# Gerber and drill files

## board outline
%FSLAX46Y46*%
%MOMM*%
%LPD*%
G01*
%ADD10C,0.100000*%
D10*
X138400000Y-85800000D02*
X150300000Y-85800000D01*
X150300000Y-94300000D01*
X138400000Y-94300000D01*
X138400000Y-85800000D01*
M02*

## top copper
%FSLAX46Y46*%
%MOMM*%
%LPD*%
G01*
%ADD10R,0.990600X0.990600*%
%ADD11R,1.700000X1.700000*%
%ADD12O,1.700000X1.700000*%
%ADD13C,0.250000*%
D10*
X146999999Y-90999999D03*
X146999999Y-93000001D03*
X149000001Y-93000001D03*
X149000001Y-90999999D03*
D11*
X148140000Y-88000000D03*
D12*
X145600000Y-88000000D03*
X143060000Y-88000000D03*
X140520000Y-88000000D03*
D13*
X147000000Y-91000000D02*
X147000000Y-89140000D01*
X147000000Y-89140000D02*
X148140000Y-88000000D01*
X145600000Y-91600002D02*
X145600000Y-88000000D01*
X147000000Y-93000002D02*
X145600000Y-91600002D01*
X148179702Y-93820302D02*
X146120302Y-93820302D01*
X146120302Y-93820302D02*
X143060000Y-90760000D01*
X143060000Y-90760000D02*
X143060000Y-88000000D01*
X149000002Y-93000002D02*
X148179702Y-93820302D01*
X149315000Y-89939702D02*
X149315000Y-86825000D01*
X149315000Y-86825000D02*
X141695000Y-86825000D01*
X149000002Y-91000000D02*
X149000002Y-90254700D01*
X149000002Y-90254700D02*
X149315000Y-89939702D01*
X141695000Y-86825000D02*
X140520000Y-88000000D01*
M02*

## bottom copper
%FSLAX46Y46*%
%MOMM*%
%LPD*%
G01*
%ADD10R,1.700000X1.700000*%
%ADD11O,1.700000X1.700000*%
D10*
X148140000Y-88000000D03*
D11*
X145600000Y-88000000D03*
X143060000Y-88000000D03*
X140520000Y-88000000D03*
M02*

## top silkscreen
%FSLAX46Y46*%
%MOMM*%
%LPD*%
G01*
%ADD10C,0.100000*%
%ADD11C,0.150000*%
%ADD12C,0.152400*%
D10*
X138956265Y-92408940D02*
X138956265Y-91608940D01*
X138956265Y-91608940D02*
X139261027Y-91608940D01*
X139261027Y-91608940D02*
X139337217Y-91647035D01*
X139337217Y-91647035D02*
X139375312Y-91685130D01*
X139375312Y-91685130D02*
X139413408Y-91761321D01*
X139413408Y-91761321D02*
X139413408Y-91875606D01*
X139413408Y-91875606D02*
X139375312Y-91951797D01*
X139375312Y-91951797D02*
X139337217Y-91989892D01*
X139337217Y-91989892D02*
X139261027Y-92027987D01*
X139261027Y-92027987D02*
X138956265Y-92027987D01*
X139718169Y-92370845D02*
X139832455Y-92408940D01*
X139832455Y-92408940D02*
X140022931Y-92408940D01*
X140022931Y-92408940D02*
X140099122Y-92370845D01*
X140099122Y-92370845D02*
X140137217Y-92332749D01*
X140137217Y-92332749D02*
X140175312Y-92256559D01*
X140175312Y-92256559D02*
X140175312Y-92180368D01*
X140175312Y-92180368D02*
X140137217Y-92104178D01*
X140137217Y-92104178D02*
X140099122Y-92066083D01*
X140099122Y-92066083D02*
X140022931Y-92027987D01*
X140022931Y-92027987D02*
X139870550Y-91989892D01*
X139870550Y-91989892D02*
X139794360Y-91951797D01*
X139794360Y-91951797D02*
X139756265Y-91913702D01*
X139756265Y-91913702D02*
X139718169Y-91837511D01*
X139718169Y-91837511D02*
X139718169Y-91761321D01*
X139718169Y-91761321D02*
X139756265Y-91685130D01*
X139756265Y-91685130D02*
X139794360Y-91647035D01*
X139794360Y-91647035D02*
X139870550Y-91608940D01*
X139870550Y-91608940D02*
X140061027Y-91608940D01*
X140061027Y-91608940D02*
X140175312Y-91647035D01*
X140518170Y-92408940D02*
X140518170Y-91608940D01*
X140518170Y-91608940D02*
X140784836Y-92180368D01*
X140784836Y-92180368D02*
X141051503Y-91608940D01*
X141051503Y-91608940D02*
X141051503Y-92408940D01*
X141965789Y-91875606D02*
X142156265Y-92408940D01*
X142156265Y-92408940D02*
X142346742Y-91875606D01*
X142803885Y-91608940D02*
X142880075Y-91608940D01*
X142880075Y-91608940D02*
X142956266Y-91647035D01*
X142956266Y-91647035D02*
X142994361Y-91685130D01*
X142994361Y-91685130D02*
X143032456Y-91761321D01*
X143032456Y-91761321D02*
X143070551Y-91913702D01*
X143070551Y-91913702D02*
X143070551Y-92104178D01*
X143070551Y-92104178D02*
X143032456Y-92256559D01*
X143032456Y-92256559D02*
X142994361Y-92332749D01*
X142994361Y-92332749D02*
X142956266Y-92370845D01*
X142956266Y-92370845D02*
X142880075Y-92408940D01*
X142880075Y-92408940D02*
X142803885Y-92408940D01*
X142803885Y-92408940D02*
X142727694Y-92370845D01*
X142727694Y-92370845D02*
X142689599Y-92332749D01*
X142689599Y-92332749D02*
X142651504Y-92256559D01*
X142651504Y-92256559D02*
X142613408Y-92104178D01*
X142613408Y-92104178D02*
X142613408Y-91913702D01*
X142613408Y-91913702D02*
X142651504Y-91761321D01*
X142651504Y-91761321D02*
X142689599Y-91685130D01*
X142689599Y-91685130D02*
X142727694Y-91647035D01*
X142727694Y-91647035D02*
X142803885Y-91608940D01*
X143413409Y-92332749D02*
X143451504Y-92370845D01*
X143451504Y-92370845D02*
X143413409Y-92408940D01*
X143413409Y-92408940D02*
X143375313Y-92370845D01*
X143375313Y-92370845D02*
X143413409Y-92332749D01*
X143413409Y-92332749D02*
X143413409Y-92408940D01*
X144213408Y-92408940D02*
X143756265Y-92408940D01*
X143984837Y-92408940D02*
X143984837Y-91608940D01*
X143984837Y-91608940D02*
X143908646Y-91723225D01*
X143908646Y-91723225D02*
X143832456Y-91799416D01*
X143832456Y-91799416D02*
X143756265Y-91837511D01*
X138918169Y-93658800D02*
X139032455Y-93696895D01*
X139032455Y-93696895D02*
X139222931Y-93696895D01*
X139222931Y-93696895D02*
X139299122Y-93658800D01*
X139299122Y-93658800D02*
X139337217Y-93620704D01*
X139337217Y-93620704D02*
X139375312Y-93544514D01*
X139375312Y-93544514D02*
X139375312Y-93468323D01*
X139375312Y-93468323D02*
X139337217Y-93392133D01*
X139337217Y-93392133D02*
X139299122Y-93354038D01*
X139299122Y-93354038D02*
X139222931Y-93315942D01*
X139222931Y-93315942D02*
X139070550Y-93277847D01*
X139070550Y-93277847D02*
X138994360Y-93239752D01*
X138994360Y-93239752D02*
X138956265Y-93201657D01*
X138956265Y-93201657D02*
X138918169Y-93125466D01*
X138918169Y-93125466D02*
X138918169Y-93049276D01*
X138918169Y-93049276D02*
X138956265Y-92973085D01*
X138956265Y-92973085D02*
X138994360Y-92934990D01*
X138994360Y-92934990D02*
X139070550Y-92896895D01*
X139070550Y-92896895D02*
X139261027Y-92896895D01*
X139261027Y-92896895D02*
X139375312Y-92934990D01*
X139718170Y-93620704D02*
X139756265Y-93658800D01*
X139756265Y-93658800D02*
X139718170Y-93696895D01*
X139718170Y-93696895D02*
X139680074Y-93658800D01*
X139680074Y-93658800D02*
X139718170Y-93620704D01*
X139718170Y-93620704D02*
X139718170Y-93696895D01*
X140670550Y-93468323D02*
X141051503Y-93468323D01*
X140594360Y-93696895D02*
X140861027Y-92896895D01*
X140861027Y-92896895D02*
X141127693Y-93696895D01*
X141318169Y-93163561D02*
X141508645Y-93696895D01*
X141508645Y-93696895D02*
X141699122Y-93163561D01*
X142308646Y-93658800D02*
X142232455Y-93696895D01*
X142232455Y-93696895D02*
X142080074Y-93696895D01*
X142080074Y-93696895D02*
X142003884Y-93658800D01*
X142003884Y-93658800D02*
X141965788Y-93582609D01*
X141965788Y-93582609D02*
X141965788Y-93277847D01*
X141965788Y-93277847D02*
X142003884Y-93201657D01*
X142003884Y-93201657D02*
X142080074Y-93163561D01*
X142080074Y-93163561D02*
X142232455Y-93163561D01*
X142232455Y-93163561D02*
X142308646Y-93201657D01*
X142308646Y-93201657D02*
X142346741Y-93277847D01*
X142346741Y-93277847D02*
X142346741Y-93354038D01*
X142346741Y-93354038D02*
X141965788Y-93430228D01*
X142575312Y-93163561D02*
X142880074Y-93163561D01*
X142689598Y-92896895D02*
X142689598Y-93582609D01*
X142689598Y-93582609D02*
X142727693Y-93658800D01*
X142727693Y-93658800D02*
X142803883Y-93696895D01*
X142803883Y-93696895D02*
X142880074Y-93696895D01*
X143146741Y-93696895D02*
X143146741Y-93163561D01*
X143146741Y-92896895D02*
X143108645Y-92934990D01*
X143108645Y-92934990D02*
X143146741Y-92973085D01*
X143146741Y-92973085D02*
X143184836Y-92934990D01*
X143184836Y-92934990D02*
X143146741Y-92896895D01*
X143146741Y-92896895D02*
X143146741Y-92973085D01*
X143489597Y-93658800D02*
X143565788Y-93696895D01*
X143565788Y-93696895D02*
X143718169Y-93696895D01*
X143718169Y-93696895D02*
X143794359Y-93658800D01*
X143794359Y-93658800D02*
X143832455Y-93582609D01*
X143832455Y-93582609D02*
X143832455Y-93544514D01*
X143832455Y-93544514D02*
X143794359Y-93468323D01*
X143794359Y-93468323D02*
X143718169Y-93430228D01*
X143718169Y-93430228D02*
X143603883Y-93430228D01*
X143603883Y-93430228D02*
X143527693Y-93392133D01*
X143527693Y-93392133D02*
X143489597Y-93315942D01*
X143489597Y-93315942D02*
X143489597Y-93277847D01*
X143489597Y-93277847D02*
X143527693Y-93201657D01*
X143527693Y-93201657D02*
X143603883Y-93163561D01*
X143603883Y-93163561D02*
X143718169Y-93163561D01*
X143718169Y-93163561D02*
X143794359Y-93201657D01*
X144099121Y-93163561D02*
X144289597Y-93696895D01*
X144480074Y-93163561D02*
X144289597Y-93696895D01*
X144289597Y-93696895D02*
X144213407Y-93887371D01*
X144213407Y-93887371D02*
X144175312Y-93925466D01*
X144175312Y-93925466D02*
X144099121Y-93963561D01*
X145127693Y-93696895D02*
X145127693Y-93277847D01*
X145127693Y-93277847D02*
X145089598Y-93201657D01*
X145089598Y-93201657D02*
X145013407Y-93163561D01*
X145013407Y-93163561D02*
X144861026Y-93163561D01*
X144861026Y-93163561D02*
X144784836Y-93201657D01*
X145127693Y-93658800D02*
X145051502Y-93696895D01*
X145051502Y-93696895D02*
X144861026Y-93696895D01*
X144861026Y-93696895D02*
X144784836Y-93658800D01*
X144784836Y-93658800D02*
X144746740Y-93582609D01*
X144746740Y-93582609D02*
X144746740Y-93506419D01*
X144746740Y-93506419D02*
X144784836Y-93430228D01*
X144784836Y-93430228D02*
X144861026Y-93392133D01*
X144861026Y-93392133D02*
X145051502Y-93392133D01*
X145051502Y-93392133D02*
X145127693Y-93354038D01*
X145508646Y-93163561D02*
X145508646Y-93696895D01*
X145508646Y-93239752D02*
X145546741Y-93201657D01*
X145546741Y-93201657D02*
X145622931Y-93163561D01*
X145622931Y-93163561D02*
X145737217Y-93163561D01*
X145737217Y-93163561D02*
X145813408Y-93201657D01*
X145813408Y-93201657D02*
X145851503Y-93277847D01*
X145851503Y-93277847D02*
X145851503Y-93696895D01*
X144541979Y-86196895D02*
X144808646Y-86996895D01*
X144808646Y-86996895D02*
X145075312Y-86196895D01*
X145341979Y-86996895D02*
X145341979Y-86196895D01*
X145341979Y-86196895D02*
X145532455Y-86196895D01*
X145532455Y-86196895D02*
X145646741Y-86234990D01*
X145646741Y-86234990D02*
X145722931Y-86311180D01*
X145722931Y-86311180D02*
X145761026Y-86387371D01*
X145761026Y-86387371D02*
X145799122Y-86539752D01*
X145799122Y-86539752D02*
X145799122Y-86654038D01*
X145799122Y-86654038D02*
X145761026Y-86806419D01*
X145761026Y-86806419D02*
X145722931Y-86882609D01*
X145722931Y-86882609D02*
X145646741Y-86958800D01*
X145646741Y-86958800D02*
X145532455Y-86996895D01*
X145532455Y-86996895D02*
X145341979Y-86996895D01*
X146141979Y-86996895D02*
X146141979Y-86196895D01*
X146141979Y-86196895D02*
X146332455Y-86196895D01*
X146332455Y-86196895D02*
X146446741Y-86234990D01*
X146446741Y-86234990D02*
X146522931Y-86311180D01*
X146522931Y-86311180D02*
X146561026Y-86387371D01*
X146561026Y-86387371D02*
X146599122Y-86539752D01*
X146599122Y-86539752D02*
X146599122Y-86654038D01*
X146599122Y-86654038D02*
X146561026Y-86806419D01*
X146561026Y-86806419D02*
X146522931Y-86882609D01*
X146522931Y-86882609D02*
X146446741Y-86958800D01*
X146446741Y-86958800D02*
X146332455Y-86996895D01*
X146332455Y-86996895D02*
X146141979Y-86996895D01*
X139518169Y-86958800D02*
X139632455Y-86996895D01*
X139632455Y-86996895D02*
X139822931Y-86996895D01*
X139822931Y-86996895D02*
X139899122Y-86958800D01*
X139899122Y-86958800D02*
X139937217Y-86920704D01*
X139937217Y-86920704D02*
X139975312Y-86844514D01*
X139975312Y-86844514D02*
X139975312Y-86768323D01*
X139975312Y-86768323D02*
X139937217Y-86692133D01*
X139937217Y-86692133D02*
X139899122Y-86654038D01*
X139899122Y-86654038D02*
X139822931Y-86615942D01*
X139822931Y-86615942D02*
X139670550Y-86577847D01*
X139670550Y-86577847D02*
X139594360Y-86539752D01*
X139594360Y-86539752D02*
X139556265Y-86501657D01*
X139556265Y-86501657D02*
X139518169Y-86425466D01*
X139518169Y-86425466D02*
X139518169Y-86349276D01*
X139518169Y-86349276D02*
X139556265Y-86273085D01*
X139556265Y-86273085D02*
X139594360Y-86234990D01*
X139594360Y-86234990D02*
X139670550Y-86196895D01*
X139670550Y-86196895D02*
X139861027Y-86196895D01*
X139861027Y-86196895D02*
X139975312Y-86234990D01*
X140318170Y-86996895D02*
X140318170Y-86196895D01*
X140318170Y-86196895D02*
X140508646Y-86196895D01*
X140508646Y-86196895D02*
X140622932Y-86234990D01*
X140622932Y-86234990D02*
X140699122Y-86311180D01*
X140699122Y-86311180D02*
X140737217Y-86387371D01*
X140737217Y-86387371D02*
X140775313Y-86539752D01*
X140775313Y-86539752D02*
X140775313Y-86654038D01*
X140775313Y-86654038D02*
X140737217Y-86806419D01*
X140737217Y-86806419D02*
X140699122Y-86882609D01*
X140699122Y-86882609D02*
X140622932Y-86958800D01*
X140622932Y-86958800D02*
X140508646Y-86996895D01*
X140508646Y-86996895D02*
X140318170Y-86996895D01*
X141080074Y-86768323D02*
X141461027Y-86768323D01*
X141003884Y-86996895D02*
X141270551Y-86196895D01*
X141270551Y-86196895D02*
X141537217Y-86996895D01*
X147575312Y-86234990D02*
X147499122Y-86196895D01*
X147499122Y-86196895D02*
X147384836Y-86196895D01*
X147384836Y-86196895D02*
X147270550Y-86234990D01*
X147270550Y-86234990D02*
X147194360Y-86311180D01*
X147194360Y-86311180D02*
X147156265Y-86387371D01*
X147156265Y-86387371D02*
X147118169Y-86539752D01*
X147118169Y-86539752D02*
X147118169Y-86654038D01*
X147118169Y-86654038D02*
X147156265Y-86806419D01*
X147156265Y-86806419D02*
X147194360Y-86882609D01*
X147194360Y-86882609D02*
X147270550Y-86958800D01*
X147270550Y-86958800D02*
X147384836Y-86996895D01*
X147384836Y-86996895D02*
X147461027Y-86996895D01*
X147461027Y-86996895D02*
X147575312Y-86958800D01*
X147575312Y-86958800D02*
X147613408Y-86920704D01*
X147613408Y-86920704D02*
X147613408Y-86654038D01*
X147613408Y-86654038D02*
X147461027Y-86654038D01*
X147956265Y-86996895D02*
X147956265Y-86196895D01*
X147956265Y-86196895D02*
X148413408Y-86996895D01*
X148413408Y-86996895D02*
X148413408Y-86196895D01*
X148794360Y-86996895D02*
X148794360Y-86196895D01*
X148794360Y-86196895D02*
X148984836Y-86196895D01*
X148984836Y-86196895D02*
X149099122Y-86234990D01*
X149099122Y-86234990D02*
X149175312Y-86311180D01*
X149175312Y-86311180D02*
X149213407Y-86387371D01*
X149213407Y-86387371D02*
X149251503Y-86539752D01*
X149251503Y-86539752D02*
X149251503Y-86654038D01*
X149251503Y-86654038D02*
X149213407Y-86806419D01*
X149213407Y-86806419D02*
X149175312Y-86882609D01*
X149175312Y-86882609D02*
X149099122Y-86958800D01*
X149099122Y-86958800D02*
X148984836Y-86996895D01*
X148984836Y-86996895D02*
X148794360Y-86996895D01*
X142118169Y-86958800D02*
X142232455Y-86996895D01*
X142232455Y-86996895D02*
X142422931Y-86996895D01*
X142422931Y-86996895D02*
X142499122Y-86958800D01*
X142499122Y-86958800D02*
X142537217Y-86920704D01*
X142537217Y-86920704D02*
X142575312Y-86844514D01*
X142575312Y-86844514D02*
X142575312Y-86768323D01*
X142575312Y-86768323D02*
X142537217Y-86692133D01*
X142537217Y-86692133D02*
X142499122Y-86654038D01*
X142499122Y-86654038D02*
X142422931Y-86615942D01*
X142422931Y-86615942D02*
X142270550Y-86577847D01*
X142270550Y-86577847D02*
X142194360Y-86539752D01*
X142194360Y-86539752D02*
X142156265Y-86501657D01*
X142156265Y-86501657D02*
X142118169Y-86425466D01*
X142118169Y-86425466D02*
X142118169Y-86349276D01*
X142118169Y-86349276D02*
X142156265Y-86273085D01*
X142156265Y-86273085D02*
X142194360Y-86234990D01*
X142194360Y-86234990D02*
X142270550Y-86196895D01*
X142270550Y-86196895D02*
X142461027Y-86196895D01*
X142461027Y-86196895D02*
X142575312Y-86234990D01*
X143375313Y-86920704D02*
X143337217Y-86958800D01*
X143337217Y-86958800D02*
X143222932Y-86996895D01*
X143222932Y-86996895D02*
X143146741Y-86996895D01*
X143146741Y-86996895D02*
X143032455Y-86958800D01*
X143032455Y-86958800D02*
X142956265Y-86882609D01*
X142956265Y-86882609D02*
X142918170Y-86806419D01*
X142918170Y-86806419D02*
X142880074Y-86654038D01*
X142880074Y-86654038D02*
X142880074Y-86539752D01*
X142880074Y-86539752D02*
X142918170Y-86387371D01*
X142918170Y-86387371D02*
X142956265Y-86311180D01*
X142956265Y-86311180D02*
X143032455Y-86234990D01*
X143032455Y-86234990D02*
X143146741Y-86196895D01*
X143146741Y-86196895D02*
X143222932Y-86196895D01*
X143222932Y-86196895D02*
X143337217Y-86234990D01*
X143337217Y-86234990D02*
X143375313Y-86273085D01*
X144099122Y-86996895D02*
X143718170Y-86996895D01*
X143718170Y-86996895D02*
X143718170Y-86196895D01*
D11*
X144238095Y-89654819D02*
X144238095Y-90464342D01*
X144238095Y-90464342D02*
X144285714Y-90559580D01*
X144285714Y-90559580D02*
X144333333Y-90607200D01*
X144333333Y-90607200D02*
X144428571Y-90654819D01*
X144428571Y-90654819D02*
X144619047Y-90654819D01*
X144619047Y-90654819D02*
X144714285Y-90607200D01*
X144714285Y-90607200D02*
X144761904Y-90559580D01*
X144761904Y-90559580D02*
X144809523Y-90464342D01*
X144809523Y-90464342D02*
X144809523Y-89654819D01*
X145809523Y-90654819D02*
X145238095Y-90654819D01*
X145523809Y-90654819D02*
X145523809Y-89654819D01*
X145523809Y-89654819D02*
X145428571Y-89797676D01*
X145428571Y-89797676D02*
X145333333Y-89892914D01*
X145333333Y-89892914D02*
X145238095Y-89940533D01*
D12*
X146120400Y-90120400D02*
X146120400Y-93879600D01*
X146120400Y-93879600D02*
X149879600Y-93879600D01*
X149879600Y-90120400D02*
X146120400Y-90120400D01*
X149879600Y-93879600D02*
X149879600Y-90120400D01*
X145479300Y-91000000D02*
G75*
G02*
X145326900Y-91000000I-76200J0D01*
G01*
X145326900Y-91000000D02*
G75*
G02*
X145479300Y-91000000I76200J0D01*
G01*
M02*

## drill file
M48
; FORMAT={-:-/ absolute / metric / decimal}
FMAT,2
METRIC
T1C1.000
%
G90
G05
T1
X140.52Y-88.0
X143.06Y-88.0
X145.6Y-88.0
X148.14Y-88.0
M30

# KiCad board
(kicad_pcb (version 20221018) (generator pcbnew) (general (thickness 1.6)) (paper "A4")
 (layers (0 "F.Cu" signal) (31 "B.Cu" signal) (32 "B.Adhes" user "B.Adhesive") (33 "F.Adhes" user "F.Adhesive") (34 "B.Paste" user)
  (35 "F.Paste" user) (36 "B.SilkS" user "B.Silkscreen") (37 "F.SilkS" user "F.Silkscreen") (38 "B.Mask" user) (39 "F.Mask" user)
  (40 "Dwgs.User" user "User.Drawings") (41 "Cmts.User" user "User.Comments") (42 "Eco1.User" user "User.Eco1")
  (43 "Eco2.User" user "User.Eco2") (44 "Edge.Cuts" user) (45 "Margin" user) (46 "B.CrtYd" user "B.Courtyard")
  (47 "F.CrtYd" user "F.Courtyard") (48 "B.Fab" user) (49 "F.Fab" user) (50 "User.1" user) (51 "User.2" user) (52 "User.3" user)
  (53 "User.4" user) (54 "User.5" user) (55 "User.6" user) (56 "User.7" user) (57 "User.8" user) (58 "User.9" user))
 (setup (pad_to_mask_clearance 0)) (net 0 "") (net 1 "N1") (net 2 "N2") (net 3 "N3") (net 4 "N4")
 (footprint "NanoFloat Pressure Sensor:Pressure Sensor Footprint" (layer "F.Cu") (at 148 92)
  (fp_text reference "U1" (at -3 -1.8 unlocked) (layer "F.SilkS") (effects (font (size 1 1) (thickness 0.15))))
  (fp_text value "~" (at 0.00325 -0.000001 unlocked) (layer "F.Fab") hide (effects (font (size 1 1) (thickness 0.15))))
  (fp_line (start -1.8796 -1.8796) (end -1.8796 1.8796) (stroke (width 0.1524) (type solid)) (layer "F.SilkS"))
  (fp_line (start -1.8796 1.8796) (end 1.8796 1.8796) (stroke (width 0.1524) (type solid)) (layer "F.SilkS"))
  (fp_line (start 1.8796 -1.8796) (end -1.8796 -1.8796) (stroke (width 0.1524) (type solid)) (layer "F.SilkS"))
  (fp_line (start 1.8796 1.8796) (end 1.8796 -1.8796) (stroke (width 0.1524) (type solid)) (layer "F.SilkS"))
  (fp_circle (center -2.5969 -1) (end -2.5207 -1) (stroke (width 0.1524) (type solid)) (fill none) (layer "F.SilkS"))
  (pad "1" smd rect (at -1.000001 -1.000001) (size 0.9906 0.9906) (layers "F.Cu" "F.Paste" "F.Mask") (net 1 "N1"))
  (pad "2" smd rect (at -1.000001 1.000001) (size 0.9906 0.9906) (layers "F.Cu" "F.Paste" "F.Mask") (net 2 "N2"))
  (pad "3" smd rect (at 1.000001 1.000001) (size 0.9906 0.9906) (layers "F.Cu" "F.Paste" "F.Mask") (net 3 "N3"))
  (pad "4" smd rect (at 1.000001 -1.000001) (size 0.9906 0.9906) (layers "F.Cu" "F.Paste" "F.Mask") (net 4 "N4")))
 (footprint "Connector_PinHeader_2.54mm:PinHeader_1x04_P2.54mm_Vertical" (layer "B.Cu") (at 148.14 88 90)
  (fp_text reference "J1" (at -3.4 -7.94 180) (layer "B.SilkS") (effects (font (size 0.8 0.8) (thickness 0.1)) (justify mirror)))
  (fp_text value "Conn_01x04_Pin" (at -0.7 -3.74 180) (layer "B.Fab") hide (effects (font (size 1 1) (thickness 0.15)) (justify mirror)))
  (pad "1" thru_hole rect (at 0 0 90) (size 1.7 1.7) (drill 1) (layers "*.Cu" "*.Mask") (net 1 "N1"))
  (pad "2" thru_hole oval (at 0 -2.54 90) (size 1.7 1.7) (drill 1) (layers "*.Cu" "*.Mask") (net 2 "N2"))
  (pad "3" thru_hole oval (at 0 -5.08 90) (size 1.7 1.7) (drill 1) (layers "*.Cu" "*.Mask") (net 3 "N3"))
  (pad "4" thru_hole oval (at 0 -7.62 90) (size 1.7 1.7) (drill 1) (layers "*.Cu" "*.Mask") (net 4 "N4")))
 (gr_rect (start 138.4 85.8) (end 150.3 94.3) (stroke (width 0.1) (type default)) (fill none) (layer "Edge.Cuts"))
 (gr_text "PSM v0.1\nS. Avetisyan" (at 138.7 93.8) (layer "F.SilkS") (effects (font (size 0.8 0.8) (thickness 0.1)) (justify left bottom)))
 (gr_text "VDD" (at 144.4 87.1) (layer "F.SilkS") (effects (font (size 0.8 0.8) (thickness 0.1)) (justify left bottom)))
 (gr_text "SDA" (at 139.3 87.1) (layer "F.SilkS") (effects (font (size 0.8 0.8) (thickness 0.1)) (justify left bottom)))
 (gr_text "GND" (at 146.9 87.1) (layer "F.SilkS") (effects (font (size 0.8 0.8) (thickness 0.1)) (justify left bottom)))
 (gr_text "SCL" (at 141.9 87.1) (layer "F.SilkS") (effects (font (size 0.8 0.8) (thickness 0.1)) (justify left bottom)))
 (segment (start 147 91) (end 147 89.14) (width 0.25) (layer "F.Cu") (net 1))
 (segment (start 147 89.14) (end 148.14 88) (width 0.25) (layer "F.Cu") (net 1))
 (segment (start 145.6 91.600002) (end 145.6 88) (width 0.25) (layer "F.Cu") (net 2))
 (segment (start 147 93.000002) (end 145.6 91.600002) (width 0.25) (layer "F.Cu") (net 2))
 (segment (start 148.179702 93.820302) (end 146.120302 93.820302) (width 0.25) (layer "F.Cu") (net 3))
 (segment (start 146.120302 93.820302) (end 143.06 90.76) (width 0.25) (layer "F.Cu") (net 3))
 (segment (start 143.06 90.76) (end 143.06 88) (width 0.25) (layer "F.Cu") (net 3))
 (segment (start 149.000002 93.000002) (end 148.179702 93.820302) (width 0.25) (layer "F.Cu") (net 3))
 (segment (start 149.315 89.939702) (end 149.315 86.825) (width 0.25) (layer "F.Cu") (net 4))
 (segment (start 149.315 86.825) (end 141.695 86.825) (width 0.25) (layer "F.Cu") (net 4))
 (segment (start 149.000002 91) (end 149.000002 90.2547) (width 0.25) (layer "F.Cu") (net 4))
 (segment (start 149.000002 90.2547) (end 149.315 89.939702) (width 0.25) (layer "F.Cu") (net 4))
 (segment (start 141.695 86.825) (end 140.52 88) (width 0.25) (layer "F.Cu") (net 4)))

